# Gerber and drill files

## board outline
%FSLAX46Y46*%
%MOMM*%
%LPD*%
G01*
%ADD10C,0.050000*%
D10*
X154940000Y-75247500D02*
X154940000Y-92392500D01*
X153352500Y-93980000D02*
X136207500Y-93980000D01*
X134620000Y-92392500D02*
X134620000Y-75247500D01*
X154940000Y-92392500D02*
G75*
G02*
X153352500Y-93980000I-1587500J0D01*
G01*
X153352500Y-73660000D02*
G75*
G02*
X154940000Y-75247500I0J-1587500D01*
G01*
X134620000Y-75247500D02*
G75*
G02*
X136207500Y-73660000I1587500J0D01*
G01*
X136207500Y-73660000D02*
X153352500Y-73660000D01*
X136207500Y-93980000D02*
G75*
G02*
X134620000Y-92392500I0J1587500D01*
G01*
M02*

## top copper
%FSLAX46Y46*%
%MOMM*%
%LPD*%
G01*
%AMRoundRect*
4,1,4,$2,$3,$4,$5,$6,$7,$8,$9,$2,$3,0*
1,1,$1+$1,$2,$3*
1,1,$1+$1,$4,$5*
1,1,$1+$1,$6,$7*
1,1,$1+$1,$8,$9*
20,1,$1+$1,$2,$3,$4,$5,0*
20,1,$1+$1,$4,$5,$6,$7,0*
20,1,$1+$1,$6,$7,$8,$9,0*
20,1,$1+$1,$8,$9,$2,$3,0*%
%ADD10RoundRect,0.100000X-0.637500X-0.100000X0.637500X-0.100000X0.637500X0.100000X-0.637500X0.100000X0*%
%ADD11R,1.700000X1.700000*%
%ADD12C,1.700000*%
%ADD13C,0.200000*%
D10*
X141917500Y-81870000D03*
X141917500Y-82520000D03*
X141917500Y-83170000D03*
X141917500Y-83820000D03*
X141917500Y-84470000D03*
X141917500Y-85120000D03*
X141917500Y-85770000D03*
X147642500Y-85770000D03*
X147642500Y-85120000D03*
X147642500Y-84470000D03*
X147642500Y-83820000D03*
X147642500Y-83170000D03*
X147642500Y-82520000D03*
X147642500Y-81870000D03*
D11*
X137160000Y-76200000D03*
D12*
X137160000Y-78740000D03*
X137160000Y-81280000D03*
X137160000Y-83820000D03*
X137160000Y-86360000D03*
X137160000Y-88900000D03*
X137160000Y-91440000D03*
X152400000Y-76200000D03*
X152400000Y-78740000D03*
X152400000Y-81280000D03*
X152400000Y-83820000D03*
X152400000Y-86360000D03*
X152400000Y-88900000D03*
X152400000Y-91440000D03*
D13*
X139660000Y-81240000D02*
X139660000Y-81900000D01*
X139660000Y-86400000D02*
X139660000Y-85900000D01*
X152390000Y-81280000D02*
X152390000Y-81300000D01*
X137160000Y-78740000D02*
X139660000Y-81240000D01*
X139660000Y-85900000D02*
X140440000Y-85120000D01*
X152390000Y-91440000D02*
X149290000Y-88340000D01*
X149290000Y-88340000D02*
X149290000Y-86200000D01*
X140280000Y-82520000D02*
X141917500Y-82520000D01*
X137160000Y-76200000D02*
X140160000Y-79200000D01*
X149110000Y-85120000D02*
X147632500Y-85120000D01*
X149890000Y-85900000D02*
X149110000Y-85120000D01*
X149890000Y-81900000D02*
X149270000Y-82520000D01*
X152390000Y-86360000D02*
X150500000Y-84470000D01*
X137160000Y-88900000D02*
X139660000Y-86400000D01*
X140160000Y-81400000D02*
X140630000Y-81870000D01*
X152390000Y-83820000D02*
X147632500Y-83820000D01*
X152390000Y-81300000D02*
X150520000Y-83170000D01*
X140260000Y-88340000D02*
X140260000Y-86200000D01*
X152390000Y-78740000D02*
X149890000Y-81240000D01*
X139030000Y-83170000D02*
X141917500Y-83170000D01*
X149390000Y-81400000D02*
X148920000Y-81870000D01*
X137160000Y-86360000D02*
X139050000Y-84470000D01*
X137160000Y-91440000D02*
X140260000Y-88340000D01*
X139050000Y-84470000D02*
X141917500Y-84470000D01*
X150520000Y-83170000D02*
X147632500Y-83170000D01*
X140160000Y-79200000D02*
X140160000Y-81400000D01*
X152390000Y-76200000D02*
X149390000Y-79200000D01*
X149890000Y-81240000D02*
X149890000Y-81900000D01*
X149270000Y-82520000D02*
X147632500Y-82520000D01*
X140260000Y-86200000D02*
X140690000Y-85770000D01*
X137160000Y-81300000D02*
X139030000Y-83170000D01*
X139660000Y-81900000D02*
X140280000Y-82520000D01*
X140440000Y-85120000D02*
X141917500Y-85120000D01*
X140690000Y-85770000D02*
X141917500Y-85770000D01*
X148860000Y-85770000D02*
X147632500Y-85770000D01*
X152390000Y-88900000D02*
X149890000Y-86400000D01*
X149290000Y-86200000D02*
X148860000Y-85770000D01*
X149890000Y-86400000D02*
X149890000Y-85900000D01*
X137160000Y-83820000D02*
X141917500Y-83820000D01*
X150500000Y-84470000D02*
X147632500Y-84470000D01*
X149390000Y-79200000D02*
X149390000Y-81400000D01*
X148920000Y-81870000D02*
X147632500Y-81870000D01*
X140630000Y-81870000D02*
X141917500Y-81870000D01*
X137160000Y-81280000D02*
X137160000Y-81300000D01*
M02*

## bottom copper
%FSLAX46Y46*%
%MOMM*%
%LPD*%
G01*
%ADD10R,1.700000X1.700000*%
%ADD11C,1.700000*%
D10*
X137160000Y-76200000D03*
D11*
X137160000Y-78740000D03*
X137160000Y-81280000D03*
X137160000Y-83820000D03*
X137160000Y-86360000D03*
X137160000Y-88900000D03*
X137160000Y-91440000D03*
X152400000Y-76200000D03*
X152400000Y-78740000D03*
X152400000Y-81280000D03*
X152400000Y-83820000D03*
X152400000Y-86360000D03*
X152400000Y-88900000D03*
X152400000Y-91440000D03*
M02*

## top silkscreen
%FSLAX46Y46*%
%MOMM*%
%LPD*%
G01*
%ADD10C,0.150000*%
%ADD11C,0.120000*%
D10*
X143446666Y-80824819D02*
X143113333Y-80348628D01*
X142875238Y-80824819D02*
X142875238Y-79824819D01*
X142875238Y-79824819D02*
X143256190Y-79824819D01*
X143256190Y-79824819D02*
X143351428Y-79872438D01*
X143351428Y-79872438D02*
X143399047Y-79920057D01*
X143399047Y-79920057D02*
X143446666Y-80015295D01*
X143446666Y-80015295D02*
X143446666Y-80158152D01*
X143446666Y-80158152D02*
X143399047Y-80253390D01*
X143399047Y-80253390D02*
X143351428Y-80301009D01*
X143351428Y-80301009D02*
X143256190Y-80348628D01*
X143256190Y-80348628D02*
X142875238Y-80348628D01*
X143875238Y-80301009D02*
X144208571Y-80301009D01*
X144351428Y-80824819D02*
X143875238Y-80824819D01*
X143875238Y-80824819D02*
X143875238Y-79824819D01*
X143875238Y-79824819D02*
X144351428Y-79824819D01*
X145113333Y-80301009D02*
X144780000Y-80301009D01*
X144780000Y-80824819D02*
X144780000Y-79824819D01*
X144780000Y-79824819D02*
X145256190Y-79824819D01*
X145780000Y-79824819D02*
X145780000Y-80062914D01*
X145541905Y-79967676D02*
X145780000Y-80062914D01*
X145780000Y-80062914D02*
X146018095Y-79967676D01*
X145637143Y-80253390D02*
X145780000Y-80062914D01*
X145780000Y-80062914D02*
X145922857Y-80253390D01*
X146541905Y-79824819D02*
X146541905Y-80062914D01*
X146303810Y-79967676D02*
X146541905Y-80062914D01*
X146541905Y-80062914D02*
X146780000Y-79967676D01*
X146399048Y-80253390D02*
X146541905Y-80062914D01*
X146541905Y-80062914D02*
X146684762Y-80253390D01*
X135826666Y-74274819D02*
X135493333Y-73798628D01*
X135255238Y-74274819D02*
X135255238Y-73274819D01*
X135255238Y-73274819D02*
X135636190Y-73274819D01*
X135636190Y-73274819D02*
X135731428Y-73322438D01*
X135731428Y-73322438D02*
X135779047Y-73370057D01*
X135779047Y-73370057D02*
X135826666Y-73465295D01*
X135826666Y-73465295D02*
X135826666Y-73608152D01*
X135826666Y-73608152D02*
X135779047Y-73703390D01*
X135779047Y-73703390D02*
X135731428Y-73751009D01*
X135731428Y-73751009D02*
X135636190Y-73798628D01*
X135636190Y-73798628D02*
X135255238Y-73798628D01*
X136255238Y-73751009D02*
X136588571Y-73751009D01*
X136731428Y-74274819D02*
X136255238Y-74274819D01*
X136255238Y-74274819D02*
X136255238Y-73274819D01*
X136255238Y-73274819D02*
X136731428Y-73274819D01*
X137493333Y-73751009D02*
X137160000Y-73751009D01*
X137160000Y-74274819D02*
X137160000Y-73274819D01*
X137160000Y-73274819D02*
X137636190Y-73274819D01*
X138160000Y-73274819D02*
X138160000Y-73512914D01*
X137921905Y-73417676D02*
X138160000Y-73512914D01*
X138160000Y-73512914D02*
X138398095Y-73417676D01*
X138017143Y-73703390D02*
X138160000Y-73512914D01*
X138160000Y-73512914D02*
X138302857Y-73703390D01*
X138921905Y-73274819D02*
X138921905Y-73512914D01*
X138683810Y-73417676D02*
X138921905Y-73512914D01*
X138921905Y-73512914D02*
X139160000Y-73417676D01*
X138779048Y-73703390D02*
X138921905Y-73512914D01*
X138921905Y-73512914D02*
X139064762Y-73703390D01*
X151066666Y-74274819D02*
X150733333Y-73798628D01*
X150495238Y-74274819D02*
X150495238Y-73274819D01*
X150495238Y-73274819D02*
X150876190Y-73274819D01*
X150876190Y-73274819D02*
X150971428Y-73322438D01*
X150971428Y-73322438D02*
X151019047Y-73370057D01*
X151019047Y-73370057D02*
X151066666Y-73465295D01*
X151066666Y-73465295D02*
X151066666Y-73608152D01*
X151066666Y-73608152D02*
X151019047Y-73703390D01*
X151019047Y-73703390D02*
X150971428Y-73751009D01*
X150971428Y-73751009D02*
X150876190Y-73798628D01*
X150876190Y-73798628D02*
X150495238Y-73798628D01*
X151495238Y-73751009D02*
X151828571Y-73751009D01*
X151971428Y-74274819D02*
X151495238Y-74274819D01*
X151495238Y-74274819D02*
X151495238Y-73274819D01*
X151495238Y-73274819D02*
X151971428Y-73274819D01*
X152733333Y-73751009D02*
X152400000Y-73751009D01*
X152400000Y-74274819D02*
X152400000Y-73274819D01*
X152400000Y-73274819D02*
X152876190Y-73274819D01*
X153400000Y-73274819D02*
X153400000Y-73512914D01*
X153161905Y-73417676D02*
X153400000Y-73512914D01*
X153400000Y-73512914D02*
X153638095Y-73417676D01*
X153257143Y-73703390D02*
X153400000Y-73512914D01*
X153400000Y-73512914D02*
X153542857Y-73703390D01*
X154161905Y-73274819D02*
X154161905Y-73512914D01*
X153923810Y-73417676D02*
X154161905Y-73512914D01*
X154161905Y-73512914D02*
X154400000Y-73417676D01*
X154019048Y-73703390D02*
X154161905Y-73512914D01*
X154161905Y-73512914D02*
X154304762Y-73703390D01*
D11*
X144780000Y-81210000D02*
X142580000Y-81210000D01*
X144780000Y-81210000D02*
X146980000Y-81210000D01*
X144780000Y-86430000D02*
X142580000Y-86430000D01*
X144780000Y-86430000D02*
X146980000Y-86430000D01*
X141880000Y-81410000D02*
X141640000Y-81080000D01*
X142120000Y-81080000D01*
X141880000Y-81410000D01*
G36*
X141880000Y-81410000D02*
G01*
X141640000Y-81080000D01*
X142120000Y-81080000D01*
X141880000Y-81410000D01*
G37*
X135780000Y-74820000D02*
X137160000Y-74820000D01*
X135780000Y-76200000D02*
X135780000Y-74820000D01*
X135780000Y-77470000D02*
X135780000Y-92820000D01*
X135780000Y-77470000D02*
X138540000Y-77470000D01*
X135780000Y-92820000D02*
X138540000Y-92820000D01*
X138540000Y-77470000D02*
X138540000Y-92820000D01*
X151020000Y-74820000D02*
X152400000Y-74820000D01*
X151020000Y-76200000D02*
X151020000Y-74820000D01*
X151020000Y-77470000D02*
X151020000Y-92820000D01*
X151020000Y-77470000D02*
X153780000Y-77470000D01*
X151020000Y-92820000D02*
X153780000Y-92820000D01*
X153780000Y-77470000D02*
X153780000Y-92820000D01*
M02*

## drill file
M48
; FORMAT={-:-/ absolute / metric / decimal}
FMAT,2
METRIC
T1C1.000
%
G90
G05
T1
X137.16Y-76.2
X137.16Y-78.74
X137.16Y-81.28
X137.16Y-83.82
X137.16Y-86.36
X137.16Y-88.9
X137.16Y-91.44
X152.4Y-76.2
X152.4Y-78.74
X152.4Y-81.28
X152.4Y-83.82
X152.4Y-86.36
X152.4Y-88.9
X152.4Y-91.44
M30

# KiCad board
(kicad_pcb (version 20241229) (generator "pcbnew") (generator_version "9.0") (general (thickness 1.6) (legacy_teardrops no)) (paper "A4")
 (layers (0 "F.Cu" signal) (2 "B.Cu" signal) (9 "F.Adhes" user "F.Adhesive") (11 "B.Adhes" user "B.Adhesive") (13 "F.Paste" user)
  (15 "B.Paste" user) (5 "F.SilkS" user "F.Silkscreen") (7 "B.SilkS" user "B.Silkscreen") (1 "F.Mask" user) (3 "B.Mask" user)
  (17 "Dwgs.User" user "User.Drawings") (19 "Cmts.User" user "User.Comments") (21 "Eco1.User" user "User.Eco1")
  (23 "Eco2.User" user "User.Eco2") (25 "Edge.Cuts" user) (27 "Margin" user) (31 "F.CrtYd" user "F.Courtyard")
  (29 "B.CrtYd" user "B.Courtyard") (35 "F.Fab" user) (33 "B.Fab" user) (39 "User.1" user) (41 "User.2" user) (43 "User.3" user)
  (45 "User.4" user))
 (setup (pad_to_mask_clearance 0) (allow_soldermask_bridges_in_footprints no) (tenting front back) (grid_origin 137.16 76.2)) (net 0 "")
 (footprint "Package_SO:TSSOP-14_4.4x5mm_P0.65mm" (layer "F.Cu") (at 144.78 83.82)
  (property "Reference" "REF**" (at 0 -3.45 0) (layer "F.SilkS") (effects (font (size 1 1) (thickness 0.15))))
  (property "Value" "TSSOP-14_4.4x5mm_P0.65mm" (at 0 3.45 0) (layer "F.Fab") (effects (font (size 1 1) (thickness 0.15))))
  (fp_line (start 0 -2.61) (end -2.2 -2.61) (stroke (width 0.12) (type solid)) (layer "F.SilkS"))
  (fp_line (start 0 -2.61) (end 2.2 -2.61) (stroke (width 0.12) (type solid)) (layer "F.SilkS"))
  (fp_line (start 0 2.61) (end -2.2 2.61) (stroke (width 0.12) (type solid)) (layer "F.SilkS"))
  (fp_line (start 0 2.61) (end 2.2 2.61) (stroke (width 0.12) (type solid)) (layer "F.SilkS"))
  (fp_poly (pts (xy -2.9 -2.41) (xy -3.14 -2.74) (xy -2.66 -2.74)) (stroke (width 0.12) (type solid)) (fill yes) (layer "F.SilkS"))
  (pad "1" smd roundrect (at -2.8625 -1.95) (size 1.475 0.4) (layers "F.Cu" "F.Mask" "F.Paste") (roundrect_rratio 0.25))
  (pad "2" smd roundrect (at -2.8625 -1.3) (size 1.475 0.4) (layers "F.Cu" "F.Mask" "F.Paste") (roundrect_rratio 0.25))
  (pad "3" smd roundrect (at -2.8625 -0.65) (size 1.475 0.4) (layers "F.Cu" "F.Mask" "F.Paste") (roundrect_rratio 0.25))
  (pad "4" smd roundrect (at -2.8625 0) (size 1.475 0.4) (layers "F.Cu" "F.Mask" "F.Paste") (roundrect_rratio 0.25))
  (pad "5" smd roundrect (at -2.8625 0.65) (size 1.475 0.4) (layers "F.Cu" "F.Mask" "F.Paste") (roundrect_rratio 0.25))
  (pad "6" smd roundrect (at -2.8625 1.3) (size 1.475 0.4) (layers "F.Cu" "F.Mask" "F.Paste") (roundrect_rratio 0.25))
  (pad "7" smd roundrect (at -2.8625 1.95) (size 1.475 0.4) (layers "F.Cu" "F.Mask" "F.Paste") (roundrect_rratio 0.25))
  (pad "8" smd roundrect (at 2.8625 1.95) (size 1.475 0.4) (layers "F.Cu" "F.Mask" "F.Paste") (roundrect_rratio 0.25))
  (pad "9" smd roundrect (at 2.8625 1.3) (size 1.475 0.4) (layers "F.Cu" "F.Mask" "F.Paste") (roundrect_rratio 0.25))
  (pad "10" smd roundrect (at 2.8625 0.65) (size 1.475 0.4) (layers "F.Cu" "F.Mask" "F.Paste") (roundrect_rratio 0.25))
  (pad "11" smd roundrect (at 2.8625 0) (size 1.475 0.4) (layers "F.Cu" "F.Mask" "F.Paste") (roundrect_rratio 0.25))
  (pad "12" smd roundrect (at 2.8625 -0.65) (size 1.475 0.4) (layers "F.Cu" "F.Mask" "F.Paste") (roundrect_rratio 0.25))
  (pad "13" smd roundrect (at 2.8625 -1.3) (size 1.475 0.4) (layers "F.Cu" "F.Mask" "F.Paste") (roundrect_rratio 0.25))
  (pad "14" smd roundrect (at 2.8625 -1.95) (size 1.475 0.4) (layers "F.Cu" "F.Mask" "F.Paste") (roundrect_rratio 0.25)))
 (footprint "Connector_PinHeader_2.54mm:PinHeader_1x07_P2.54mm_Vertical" (layer "F.Cu") (at 137.16 76.2)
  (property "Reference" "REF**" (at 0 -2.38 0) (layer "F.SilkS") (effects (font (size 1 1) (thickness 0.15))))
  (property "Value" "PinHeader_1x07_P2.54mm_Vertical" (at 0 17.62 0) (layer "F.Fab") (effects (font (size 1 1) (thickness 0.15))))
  (fp_line (start -1.38 -1.38) (end 0 -1.38) (stroke (width 0.12) (type solid)) (layer "F.SilkS"))
  (fp_line (start -1.38 0) (end -1.38 -1.38) (stroke (width 0.12) (type solid)) (layer "F.SilkS"))
  (fp_line (start -1.38 1.27) (end -1.38 16.62) (stroke (width 0.12) (type solid)) (layer "F.SilkS"))
  (fp_line (start -1.38 1.27) (end 1.38 1.27) (stroke (width 0.12) (type solid)) (layer "F.SilkS"))
  (fp_line (start -1.38 16.62) (end 1.38 16.62) (stroke (width 0.12) (type solid)) (layer "F.SilkS"))
  (fp_line (start 1.38 1.27) (end 1.38 16.62) (stroke (width 0.12) (type solid)) (layer "F.SilkS"))
  (pad "1" thru_hole rect (at 0 0) (size 1.7 1.7) (drill 1) (layers "*.Cu" "*.Mask") (remove_unused_layers no))
  (pad "2" thru_hole circle (at 0 2.54) (size 1.7 1.7) (drill 1) (layers "*.Cu" "*.Mask") (remove_unused_layers no))
  (pad "3" thru_hole circle (at 0 5.08) (size 1.7 1.7) (drill 1) (layers "*.Cu" "*.Mask") (remove_unused_layers no))
  (pad "4" thru_hole circle (at 0 7.62) (size 1.7 1.7) (drill 1) (layers "*.Cu" "*.Mask") (remove_unused_layers no))
  (pad "5" thru_hole circle (at 0 10.16) (size 1.7 1.7) (drill 1) (layers "*.Cu" "*.Mask") (remove_unused_layers no))
  (pad "6" thru_hole circle (at 0 12.7) (size 1.7 1.7) (drill 1) (layers "*.Cu" "*.Mask") (remove_unused_layers no))
  (pad "7" thru_hole circle (at 0 15.24) (size 1.7 1.7) (drill 1) (layers "*.Cu" "*.Mask") (remove_unused_layers no)))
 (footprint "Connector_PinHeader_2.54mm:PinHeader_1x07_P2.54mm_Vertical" (layer "F.Cu") (at 152.4 76.2)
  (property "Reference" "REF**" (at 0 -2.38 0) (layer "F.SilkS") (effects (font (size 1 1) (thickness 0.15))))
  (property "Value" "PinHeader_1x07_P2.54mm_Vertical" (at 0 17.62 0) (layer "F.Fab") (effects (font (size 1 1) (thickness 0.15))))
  (fp_line (start -1.38 -1.38) (end 0 -1.38) (stroke (width 0.12) (type solid)) (layer "F.SilkS"))
  (fp_line (start -1.38 0) (end -1.38 -1.38) (stroke (width 0.12) (type solid)) (layer "F.SilkS"))
  (fp_line (start -1.38 1.27) (end -1.38 16.62) (stroke (width 0.12) (type solid)) (layer "F.SilkS"))
  (fp_line (start -1.38 1.27) (end 1.38 1.27) (stroke (width 0.12) (type solid)) (layer "F.SilkS"))
  (fp_line (start -1.38 16.62) (end 1.38 16.62) (stroke (width 0.12) (type solid)) (layer "F.SilkS"))
  (fp_line (start 1.38 1.27) (end 1.38 16.62) (stroke (width 0.12) (type solid)) (layer "F.SilkS"))
  (pad "1" thru_hole circle (at 0 0) (size 1.7 1.7) (drill 1) (layers "*.Cu" "*.Mask") (remove_unused_layers no))
  (pad "2" thru_hole circle (at 0 2.54) (size 1.7 1.7) (drill 1) (layers "*.Cu" "*.Mask") (remove_unused_layers no))
  (pad "3" thru_hole circle (at 0 5.08) (size 1.7 1.7) (drill 1) (layers "*.Cu" "*.Mask") (remove_unused_layers no))
  (pad "4" thru_hole circle (at 0 7.62) (size 1.7 1.7) (drill 1) (layers "*.Cu" "*.Mask") (remove_unused_layers no))
  (pad "5" thru_hole circle (at 0 10.16) (size 1.7 1.7) (drill 1) (layers "*.Cu" "*.Mask") (remove_unused_layers no))
  (pad "6" thru_hole circle (at 0 12.7) (size 1.7 1.7) (drill 1) (layers "*.Cu" "*.Mask") (remove_unused_layers no))
  (pad "7" thru_hole circle (at 0 15.24) (size 1.7 1.7) (drill 1) (layers "*.Cu" "*.Mask") (remove_unused_layers no)))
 (gr_line (start 154.94 75.2475) (end 154.94 92.3925) (stroke (width 0.05) (type default)) (layer "Edge.Cuts"))
 (gr_line (start 153.3525 93.98) (end 136.2075 93.98) (stroke (width 0.05) (type default)) (layer "Edge.Cuts"))
 (gr_line (start 134.62 92.3925) (end 134.62 75.2475) (stroke (width 0.05) (type default)) (layer "Edge.Cuts"))
 (gr_arc (start 154.94 92.3925) (mid 154.475032 93.515032) (end 153.3525 93.98) (stroke (width 0.05) (type default)) (layer "Edge.Cuts"))
 (gr_arc (start 153.3525 73.66) (mid 154.475032 74.124968) (end 154.94 75.2475) (stroke (width 0.05) (type default)) (layer "Edge.Cuts"))
 (gr_arc (start 134.62 75.2475) (mid 135.084968 74.124968) (end 136.2075 73.66) (stroke (width 0.05) (type default)) (layer "Edge.Cuts"))
 (gr_line (start 136.2075 73.66) (end 153.3525 73.66) (stroke (width 0.05) (type default)) (layer "Edge.Cuts"))
 (gr_arc (start 136.2075 93.98) (mid 135.084968 93.515032) (end 134.62 92.3925) (stroke (width 0.05) (type default)) (layer "Edge.Cuts"))
 (segment (start 139.66 81.24) (end 139.66 81.9) (width 0.2) (layer "F.Cu") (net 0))
 (segment (start 139.66 86.4) (end 139.66 85.9) (width 0.2) (layer "F.Cu") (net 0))
 (segment (start 152.39 81.28) (end 152.39 81.3) (width 0.2) (layer "F.Cu") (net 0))
 (segment (start 137.16 78.74) (end 139.66 81.24) (width 0.2) (layer "F.Cu") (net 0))
 (segment (start 139.66 85.9) (end 140.44 85.12) (width 0.2) (layer "F.Cu") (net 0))
 (segment (start 152.39 91.44) (end 149.29 88.34) (width 0.2) (layer "F.Cu") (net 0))
 (segment (start 149.29 88.34) (end 149.29 86.2) (width 0.2) (layer "F.Cu") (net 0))
 (segment (start 140.28 82.52) (end 141.9175 82.52) (width 0.2) (layer "F.Cu") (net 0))
 (segment (start 137.16 76.2) (end 140.16 79.2) (width 0.2) (layer "F.Cu") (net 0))
 (segment (start 149.11 85.12) (end 147.6325 85.12) (width 0.2) (layer "F.Cu") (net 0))
 (segment (start 149.89 85.9) (end 149.11 85.12) (width 0.2) (layer "F.Cu") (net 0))
 (segment (start 149.89 81.9) (end 149.27 82.52) (width 0.2) (layer "F.Cu") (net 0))
 (segment (start 152.39 86.36) (end 150.5 84.47) (width 0.2) (layer "F.Cu") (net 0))
 (segment (start 137.16 88.9) (end 139.66 86.4) (width 0.2) (layer "F.Cu") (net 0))
 (segment (start 140.16 81.4) (end 140.63 81.87) (width 0.2) (layer "F.Cu") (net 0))
 (segment (start 152.39 83.82) (end 147.6325 83.82) (width 0.2) (layer "F.Cu") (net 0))
 (segment (start 152.39 81.3) (end 150.52 83.17) (width 0.2) (layer "F.Cu") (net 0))
 (segment (start 140.26 88.34) (end 140.26 86.2) (width 0.2) (layer "F.Cu") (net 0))
 (segment (start 152.39 78.74) (end 149.89 81.24) (width 0.2) (layer "F.Cu") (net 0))
 (segment (start 139.03 83.17) (end 141.9175 83.17) (width 0.2) (layer "F.Cu") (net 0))
 (segment (start 149.39 81.4) (end 148.92 81.87) (width 0.2) (layer "F.Cu") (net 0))
 (segment (start 137.16 86.36) (end 139.05 84.47) (width 0.2) (layer "F.Cu") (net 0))
 (segment (start 137.16 91.44) (end 140.26 88.34) (width 0.2) (layer "F.Cu") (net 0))
 (segment (start 139.05 84.47) (end 141.9175 84.47) (width 0.2) (layer "F.Cu") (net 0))
 (segment (start 150.52 83.17) (end 147.6325 83.17) (width 0.2) (layer "F.Cu") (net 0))
 (segment (start 140.16 79.2) (end 140.16 81.4) (width 0.2) (layer "F.Cu") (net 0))
 (segment (start 152.39 76.2) (end 149.39 79.2) (width 0.2) (layer "F.Cu") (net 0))
 (segment (start 149.89 81.24) (end 149.89 81.9) (width 0.2) (layer "F.Cu") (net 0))
 (segment (start 149.27 82.52) (end 147.6325 82.52) (width 0.2) (layer "F.Cu") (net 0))
 (segment (start 140.26 86.2) (end 140.69 85.77) (width 0.2) (layer "F.Cu") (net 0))
 (segment (start 137.16 81.3) (end 139.03 83.17) (width 0.2) (layer "F.Cu") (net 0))
 (segment (start 139.66 81.9) (end 140.28 82.52) (width 0.2) (layer "F.Cu") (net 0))
 (segment (start 140.44 85.12) (end 141.9175 85.12) (width 0.2) (layer "F.Cu") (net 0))
 (segment (start 140.69 85.77) (end 141.9175 85.77) (width 0.2) (layer "F.Cu") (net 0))
 (segment (start 148.86 85.77) (end 147.6325 85.77) (width 0.2) (layer "F.Cu") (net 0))
 (segment (start 152.39 88.9) (end 149.89 86.4) (width 0.2) (layer "F.Cu") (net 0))
 (segment (start 149.29 86.2) (end 148.86 85.77) (width 0.2) (layer "F.Cu") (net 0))
 (segment (start 149.89 86.4) (end 149.89 85.9) (width 0.2) (layer "F.Cu") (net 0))
 (segment (start 137.16 83.82) (end 141.9175 83.82) (width 0.2) (layer "F.Cu") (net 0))
 (segment (start 150.5 84.47) (end 147.6325 84.47) (width 0.2) (layer "F.Cu") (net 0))
 (segment (start 149.39 79.2) (end 149.39 81.4) (width 0.2) (layer "F.Cu") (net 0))
 (segment (start 148.92 81.87) (end 147.6325 81.87) (width 0.2) (layer "F.Cu") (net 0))
 (segment (start 140.63 81.87) (end 141.9175 81.87) (width 0.2) (layer "F.Cu") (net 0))
 (segment (start 137.16 81.28) (end 137.16 81.3) (width 0.2) (layer "F.Cu") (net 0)))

